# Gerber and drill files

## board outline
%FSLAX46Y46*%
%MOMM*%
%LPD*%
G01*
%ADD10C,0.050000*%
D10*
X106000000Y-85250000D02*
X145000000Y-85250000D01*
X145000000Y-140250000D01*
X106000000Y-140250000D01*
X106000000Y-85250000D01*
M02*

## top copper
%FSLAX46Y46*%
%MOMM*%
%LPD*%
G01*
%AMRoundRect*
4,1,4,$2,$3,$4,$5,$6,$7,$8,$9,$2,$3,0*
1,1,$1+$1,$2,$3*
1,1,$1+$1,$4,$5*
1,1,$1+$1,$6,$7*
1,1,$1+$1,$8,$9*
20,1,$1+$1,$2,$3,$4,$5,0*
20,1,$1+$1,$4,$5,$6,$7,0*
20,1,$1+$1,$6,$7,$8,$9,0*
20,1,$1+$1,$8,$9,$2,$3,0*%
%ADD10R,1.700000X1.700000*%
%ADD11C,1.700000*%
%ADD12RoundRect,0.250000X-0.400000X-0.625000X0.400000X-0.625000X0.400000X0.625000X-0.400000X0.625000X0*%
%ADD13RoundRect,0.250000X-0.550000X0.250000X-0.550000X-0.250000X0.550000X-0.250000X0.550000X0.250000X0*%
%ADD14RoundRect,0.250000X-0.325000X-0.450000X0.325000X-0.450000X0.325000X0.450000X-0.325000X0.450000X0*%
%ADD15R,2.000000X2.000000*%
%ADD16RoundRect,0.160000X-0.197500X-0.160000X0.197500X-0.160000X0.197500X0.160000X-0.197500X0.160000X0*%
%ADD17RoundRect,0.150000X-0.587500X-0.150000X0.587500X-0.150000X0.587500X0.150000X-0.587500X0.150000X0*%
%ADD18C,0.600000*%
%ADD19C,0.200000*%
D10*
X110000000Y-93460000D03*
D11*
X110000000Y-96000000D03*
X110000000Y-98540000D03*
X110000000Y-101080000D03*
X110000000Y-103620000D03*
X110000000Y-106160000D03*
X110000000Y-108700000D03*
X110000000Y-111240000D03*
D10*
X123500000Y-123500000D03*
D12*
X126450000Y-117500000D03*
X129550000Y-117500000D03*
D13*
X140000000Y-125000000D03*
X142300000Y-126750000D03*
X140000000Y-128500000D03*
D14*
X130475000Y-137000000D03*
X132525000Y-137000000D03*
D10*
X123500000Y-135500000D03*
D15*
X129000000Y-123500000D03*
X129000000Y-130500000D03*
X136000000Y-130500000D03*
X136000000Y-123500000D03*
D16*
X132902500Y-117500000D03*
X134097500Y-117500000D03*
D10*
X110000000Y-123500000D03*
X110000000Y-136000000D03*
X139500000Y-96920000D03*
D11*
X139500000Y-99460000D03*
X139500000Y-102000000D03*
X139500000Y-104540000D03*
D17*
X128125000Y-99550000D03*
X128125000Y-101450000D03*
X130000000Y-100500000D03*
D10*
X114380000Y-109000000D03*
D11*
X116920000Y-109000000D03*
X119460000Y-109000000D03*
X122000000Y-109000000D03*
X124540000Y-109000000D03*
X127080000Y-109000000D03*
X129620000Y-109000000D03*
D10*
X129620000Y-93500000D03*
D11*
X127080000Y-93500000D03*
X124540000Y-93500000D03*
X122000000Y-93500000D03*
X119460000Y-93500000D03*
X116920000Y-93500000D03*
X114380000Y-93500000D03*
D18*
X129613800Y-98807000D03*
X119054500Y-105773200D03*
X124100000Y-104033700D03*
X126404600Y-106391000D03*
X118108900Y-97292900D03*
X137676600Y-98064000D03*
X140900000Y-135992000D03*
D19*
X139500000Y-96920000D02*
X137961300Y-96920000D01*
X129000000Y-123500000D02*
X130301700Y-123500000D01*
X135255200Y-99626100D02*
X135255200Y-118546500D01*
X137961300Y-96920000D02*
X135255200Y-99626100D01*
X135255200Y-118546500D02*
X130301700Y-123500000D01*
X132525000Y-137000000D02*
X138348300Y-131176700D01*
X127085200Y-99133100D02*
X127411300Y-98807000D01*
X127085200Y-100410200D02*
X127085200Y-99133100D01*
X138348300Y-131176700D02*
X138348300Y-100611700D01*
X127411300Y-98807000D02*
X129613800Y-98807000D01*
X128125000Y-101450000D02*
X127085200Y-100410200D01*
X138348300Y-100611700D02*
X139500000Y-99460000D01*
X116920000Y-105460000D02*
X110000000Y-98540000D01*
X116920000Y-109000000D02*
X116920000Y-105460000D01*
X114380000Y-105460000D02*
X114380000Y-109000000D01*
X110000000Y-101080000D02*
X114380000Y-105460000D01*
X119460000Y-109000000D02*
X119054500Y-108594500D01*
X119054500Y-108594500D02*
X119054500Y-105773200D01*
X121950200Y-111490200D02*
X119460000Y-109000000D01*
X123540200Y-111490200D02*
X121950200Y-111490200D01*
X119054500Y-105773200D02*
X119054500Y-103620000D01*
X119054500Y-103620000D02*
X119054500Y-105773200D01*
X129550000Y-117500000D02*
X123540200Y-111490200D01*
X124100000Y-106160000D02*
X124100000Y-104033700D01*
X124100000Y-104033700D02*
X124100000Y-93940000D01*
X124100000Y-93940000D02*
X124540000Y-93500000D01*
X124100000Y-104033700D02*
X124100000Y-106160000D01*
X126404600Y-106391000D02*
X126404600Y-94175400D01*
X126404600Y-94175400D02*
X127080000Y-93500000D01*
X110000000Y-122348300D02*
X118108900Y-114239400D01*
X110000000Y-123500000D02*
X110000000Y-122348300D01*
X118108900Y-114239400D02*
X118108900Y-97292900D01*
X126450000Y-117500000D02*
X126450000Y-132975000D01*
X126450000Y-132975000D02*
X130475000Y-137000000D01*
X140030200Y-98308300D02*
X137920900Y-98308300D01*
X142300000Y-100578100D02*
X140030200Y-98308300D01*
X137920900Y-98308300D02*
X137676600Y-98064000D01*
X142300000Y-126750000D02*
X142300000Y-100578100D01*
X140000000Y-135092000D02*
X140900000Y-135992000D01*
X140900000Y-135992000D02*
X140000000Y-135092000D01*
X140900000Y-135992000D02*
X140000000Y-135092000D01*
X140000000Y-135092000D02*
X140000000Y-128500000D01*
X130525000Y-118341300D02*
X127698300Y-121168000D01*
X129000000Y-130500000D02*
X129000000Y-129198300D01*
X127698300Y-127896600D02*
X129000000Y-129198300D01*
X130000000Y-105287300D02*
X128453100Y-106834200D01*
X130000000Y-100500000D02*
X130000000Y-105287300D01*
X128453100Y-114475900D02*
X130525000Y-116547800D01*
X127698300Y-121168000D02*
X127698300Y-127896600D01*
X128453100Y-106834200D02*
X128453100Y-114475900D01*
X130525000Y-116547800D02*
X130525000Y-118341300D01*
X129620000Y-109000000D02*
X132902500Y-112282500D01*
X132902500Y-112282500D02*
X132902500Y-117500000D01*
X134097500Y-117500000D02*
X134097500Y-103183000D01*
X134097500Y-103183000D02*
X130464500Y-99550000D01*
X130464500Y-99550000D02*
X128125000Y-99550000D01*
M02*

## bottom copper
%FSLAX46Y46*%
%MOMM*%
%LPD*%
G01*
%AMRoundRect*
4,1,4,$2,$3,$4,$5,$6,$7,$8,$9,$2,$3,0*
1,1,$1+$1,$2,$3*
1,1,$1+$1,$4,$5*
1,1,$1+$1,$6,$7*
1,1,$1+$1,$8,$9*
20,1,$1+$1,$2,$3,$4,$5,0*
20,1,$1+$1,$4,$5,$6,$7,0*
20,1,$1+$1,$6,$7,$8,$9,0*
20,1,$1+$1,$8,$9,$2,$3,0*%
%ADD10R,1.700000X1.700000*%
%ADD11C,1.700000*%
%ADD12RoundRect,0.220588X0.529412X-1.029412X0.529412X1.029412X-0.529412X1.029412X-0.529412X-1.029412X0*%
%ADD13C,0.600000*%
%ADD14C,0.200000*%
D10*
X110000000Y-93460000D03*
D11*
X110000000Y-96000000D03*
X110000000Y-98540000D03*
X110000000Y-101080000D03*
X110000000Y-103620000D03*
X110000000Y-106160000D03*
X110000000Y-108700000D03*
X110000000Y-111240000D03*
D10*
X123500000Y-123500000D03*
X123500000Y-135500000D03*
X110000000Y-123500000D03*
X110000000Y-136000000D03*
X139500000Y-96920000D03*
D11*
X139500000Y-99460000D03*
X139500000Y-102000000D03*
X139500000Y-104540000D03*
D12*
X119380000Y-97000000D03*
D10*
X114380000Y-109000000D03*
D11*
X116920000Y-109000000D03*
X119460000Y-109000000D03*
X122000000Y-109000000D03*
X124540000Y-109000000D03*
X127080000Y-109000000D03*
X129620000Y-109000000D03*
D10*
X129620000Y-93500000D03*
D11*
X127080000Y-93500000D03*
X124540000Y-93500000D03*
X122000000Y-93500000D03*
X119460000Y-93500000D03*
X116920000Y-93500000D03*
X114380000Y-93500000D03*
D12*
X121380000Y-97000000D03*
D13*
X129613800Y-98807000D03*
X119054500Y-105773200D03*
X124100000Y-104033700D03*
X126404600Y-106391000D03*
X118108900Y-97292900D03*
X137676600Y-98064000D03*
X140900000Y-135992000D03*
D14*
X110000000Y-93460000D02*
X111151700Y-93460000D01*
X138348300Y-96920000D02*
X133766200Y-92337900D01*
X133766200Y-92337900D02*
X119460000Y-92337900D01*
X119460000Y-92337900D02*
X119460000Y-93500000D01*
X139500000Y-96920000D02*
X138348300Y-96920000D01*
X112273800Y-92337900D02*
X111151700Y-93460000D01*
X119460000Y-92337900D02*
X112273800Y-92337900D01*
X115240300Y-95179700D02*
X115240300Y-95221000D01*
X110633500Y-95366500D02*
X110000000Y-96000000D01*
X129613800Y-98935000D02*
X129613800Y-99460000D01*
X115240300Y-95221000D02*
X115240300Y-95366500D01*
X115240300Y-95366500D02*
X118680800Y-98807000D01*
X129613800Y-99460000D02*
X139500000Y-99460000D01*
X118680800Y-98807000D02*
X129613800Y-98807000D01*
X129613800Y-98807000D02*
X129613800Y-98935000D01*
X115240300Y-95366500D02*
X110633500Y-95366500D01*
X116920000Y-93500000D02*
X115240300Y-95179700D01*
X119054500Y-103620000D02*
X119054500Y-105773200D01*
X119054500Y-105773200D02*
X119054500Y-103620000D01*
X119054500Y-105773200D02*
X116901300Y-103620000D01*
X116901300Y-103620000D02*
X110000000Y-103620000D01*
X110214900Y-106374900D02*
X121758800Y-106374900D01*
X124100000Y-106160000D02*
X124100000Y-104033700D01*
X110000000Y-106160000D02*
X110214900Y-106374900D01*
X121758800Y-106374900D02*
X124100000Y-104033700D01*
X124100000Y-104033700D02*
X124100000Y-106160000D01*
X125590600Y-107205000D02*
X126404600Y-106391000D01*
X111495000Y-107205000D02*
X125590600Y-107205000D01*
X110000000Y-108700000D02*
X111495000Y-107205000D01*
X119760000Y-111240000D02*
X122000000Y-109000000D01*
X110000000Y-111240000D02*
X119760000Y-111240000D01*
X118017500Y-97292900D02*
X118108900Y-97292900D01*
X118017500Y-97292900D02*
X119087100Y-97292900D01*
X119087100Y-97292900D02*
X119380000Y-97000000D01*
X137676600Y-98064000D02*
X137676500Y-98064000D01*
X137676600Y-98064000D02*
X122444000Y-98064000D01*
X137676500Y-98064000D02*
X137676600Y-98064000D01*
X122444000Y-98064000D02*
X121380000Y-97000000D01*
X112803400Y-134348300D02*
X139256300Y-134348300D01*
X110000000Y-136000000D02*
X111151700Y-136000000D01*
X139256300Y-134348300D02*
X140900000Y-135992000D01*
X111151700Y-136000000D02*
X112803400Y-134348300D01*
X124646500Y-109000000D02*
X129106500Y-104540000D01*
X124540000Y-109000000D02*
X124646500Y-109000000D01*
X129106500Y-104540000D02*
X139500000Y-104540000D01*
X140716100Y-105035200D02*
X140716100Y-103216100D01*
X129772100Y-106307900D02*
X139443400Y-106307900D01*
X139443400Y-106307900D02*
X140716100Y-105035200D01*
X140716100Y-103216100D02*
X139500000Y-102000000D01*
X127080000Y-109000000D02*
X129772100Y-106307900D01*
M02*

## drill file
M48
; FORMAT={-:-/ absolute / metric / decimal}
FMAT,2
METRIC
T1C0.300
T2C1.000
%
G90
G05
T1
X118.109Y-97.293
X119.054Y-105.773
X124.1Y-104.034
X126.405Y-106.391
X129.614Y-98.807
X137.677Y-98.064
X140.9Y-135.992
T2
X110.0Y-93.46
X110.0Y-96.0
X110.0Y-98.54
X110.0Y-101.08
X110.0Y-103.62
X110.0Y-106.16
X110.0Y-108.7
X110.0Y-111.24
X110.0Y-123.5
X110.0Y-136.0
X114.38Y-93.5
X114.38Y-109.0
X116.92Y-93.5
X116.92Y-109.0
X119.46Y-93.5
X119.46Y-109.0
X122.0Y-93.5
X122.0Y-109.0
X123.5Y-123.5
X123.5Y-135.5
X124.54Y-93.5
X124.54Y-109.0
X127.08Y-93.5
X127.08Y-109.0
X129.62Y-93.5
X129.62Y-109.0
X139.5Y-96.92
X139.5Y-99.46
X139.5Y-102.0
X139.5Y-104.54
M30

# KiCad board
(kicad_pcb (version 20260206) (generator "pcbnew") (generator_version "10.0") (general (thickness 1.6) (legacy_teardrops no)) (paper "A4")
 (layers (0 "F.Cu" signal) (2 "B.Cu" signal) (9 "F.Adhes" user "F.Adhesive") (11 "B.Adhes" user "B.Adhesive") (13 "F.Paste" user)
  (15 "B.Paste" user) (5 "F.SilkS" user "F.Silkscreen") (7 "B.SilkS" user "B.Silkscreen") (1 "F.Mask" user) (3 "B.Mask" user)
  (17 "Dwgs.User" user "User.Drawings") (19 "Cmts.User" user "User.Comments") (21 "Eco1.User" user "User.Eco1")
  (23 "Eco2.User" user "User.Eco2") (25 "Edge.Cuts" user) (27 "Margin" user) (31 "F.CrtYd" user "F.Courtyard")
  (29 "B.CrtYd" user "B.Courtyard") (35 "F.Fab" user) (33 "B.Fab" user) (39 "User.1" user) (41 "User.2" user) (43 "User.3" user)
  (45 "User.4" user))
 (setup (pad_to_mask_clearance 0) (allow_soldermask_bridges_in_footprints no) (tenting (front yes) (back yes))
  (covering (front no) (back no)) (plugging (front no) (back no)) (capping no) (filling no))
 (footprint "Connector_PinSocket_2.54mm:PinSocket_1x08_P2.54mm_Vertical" (layer "F.Cu") (at 110 93.46)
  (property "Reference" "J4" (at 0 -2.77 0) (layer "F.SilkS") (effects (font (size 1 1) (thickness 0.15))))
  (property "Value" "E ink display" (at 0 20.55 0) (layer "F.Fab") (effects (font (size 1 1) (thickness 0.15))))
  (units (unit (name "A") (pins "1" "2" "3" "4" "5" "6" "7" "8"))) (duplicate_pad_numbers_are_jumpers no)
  (pad "1" thru_hole rect (at 0 0) (size 1.7 1.7) (drill 1) (layers "*.Cu" "*.Mask") (remove_unused_layers no) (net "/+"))
  (pad "2" thru_hole circle (at 0 2.54) (size 1.7 1.7) (drill 1) (layers "*.Cu" "*.Mask") (remove_unused_layers no) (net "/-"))
  (pad "3" thru_hole circle (at 0 5.08) (size 1.7 1.7) (drill 1) (layers "*.Cu" "*.Mask") (remove_unused_layers no) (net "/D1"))
  (pad "4" thru_hole circle (at 0 7.62) (size 1.7 1.7) (drill 1) (layers "*.Cu" "*.Mask") (remove_unused_layers no) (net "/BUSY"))
  (pad "5" thru_hole circle (at 0 10.16) (size 1.7 1.7) (drill 1) (layers "*.Cu" "*.Mask") (remove_unused_layers no) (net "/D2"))
  (pad "6" thru_hole circle (at 0 12.7) (size 1.7 1.7) (drill 1) (layers "*.Cu" "*.Mask") (remove_unused_layers no) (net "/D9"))
  (pad "7" thru_hole circle (at 0 15.24) (size 1.7 1.7) (drill 1) (layers "*.Cu" "*.Mask") (remove_unused_layers no) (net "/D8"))
  (pad "8" thru_hole circle (at 0 17.78) (size 1.7 1.7) (drill 1) (layers "*.Cu" "*.Mask") (remove_unused_layers no) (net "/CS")))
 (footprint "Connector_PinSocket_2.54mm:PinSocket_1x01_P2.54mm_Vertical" (layer "F.Cu") (at 123.5 123.5)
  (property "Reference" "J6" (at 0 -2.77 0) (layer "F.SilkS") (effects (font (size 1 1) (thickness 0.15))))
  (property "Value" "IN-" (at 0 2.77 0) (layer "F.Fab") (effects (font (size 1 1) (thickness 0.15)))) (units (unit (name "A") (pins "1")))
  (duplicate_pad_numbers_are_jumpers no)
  (pad "1" thru_hole rect (at 0 0) (size 1.7 1.7) (drill 1) (layers "*.Cu" "*.Mask") (remove_unused_layers no)
   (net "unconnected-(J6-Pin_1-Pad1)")))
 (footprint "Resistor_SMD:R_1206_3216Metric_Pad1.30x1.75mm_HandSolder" (layer "F.Cu") (at 128 117.5)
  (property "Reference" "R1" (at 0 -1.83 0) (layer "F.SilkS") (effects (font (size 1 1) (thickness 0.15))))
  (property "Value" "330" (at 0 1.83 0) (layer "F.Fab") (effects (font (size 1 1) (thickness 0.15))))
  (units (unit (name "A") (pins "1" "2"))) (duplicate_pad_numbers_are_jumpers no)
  (pad "1" smd roundrect (at -1.55 0) (size 1.3 1.75) (layers "F.Cu" "F.Mask" "F.Paste") (roundrect_rratio 0.192308) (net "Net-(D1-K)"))
  (pad "2" smd roundrect (at 1.55 0) (size 1.3 1.75) (layers "F.Cu" "F.Mask" "F.Paste") (roundrect_rratio 0.192308) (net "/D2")))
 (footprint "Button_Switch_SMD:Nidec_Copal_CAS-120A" (layer "F.Cu") (at 141.15 126.75)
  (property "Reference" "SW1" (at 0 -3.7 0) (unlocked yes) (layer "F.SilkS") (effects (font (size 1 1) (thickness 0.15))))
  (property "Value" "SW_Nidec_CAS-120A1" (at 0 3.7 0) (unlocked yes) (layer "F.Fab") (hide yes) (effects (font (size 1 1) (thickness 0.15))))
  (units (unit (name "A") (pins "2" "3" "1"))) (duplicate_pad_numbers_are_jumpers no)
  (pad "1" smd roundrect (at -1.15 -1.75 270) (size 1 1.6) (layers "F.Cu" "F.Mask" "F.Paste") (roundrect_rratio 0.25)
   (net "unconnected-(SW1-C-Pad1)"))
  (pad "2" smd roundrect (at 1.15 0 270) (size 1 1.6) (layers "F.Cu" "F.Mask" "F.Paste") (roundrect_rratio 0.25) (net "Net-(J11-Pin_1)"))
  (pad "3" smd roundrect (at -1.15 1.75 270) (size 1 1.6) (layers "F.Cu" "F.Mask" "F.Paste") (roundrect_rratio 0.25) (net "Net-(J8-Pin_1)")))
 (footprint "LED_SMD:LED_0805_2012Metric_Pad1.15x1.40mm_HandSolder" (layer "F.Cu") (at 131.5 137)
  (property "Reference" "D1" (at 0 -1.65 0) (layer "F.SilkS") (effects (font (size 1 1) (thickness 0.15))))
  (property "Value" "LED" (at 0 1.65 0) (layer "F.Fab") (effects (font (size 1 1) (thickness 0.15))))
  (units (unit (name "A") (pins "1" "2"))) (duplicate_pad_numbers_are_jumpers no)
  (pad "1" smd roundrect (at -1.025 0) (size 1.15 1.4) (layers "F.Cu" "F.Mask" "F.Paste") (roundrect_rratio 0.217391) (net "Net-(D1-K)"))
  (pad "2" smd roundrect (at 1.025 0) (size 1.15 1.4) (layers "F.Cu" "F.Mask" "F.Paste") (roundrect_rratio 0.217391) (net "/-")))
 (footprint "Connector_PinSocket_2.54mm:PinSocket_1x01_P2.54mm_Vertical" (layer "F.Cu") (at 123.5 135.5)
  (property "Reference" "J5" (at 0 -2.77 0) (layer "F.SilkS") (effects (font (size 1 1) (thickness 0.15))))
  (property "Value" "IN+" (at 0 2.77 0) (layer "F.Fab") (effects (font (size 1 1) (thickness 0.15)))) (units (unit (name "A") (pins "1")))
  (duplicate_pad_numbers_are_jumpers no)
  (pad "1" thru_hole rect (at 0 0) (size 1.7 1.7) (drill 1) (layers "*.Cu" "*.Mask") (remove_unused_layers no)
   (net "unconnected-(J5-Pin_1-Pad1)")))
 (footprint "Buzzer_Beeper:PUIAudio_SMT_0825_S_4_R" (layer "F.Cu") (at 132.5 127)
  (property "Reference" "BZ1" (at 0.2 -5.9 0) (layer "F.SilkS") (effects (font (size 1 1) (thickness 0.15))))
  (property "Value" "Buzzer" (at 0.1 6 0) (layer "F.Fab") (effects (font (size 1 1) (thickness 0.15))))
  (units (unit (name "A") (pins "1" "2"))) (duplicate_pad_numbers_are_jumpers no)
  (pad "1" smd rect (at -3.5 -3.5 270) (size 2 2) (layers "F.Cu" "F.Mask" "F.Paste") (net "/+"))
  (pad "2" smd rect (at -3.5 3.5 270) (size 2 2) (layers "F.Cu" "F.Mask" "F.Paste") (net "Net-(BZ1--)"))
  (pad "3" smd rect (at 3.5 3.5 270) (size 2 2) (layers "F.Cu" "F.Mask" "F.Paste"))
  (pad "4" smd rect (at 3.5 -3.5 270) (size 2 2) (layers "F.Cu" "F.Mask" "F.Paste")))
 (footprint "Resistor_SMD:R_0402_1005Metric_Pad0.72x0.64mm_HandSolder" (layer "F.Cu") (at 133.5 117.5)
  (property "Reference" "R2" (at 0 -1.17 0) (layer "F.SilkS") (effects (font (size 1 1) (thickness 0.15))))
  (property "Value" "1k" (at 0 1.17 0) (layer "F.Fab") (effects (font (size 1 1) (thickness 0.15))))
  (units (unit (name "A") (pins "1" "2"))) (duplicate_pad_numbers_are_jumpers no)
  (pad "1" smd roundrect (at -0.5975 0) (size 0.715 0.64) (layers "F.Cu" "F.Mask" "F.Paste") (roundrect_rratio 0.25) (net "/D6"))
  (pad "2" smd roundrect (at 0.5975 0) (size 0.715 0.64) (layers "F.Cu" "F.Mask" "F.Paste") (roundrect_rratio 0.25) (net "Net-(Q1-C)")))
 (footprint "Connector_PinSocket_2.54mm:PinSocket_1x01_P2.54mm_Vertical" (layer "F.Cu") (at 110 123.5)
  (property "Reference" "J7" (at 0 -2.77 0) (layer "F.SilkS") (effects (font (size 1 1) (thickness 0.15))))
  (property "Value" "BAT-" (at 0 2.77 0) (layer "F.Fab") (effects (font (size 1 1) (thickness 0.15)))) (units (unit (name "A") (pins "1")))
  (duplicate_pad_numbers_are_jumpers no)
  (pad "1" thru_hole rect (at 0 0) (size 1.7 1.7) (drill 1) (layers "*.Cu" "*.Mask") (remove_unused_layers no) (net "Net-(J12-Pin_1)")))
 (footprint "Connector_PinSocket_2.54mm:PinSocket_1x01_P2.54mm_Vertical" (layer "F.Cu") (at 110 136)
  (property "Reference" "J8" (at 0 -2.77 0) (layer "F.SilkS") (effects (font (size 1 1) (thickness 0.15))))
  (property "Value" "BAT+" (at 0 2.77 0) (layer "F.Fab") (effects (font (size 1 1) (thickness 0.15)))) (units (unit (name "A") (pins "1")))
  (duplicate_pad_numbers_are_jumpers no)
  (pad "1" thru_hole rect (at 0 0) (size 1.7 1.7) (drill 1) (layers "*.Cu" "*.Mask") (remove_unused_layers no) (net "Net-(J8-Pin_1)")))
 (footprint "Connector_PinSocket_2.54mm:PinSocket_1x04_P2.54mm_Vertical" (layer "F.Cu") (at 139.5 96.92)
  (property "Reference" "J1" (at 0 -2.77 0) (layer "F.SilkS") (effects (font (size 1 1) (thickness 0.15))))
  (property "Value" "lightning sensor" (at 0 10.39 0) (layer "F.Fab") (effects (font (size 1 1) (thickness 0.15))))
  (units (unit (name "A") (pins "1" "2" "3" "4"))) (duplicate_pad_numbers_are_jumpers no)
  (pad "1" thru_hole rect (at 0 0) (size 1.7 1.7) (drill 1) (layers "*.Cu" "*.Mask") (remove_unused_layers no) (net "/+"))
  (pad "2" thru_hole circle (at 0 2.54) (size 1.7 1.7) (drill 1) (layers "*.Cu" "*.Mask") (remove_unused_layers no) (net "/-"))
  (pad "3" thru_hole circle (at 0 5.08) (size 1.7 1.7) (drill 1) (layers "*.Cu" "*.Mask") (remove_unused_layers no) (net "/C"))
  (pad "4" thru_hole circle (at 0 7.62) (size 1.7 1.7) (drill 1) (layers "*.Cu" "*.Mask") (remove_unused_layers no) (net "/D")))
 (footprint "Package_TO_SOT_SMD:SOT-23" (layer "F.Cu") (at 129.0625 100.5)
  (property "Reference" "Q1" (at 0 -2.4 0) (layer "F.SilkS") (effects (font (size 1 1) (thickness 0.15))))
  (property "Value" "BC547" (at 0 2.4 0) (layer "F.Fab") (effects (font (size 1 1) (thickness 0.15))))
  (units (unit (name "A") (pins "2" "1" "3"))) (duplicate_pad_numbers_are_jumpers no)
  (pad "1" smd roundrect (at -0.9375 -0.95) (size 1.475 0.6) (layers "F.Cu" "F.Mask" "F.Paste") (roundrect_rratio 0.25) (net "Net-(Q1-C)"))
  (pad "2" smd roundrect (at -0.9375 0.95) (size 1.475 0.6) (layers "F.Cu" "F.Mask" "F.Paste") (roundrect_rratio 0.25) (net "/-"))
  (pad "3" smd roundrect (at 0.9375 0) (size 1.475 0.6) (layers "F.Cu" "F.Mask" "F.Paste") (roundrect_rratio 0.25) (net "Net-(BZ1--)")))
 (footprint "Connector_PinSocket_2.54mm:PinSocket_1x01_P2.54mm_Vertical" (layer "B.Cu") (at 119.38 97 90)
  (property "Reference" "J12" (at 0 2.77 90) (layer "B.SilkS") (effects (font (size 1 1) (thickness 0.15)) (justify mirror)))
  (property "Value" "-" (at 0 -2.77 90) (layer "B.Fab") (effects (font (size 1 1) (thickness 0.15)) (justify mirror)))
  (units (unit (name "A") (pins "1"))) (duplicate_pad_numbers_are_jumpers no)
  (pad "1" smd roundrect (at 0 0 90) (size 2.5 1.5) (layers "B.Cu" "B.Mask" "B.Paste") (roundrect_rratio 0.1470588235)
   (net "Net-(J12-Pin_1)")))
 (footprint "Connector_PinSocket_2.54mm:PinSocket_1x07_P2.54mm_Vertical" (layer "B.Cu") (at 114.38 109 -90)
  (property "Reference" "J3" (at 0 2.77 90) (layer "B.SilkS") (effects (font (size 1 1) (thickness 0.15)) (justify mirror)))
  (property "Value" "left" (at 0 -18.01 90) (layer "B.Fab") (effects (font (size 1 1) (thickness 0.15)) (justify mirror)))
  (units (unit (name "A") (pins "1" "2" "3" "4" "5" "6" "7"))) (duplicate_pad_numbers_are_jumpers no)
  (pad "1" thru_hole rect (at 0 0 270) (size 1.7 1.7) (drill 1) (layers "*.Cu" "*.Mask") (remove_unused_layers no) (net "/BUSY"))
  (pad "2" thru_hole circle (at 0 -2.54 270) (size 1.7 1.7) (drill 1) (layers "*.Cu" "*.Mask") (remove_unused_layers no) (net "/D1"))
  (pad "3" thru_hole circle (at 0 -5.08 270) (size 1.7 1.7) (drill 1) (layers "*.Cu" "*.Mask") (remove_unused_layers no) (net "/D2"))
  (pad "4" thru_hole circle (at 0 -7.62 270) (size 1.7 1.7) (drill 1) (layers "*.Cu" "*.Mask") (remove_unused_layers no) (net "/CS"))
  (pad "5" thru_hole circle (at 0 -10.16 270) (size 1.7 1.7) (drill 1) (layers "*.Cu" "*.Mask") (remove_unused_layers no) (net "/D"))
  (pad "6" thru_hole circle (at 0 -12.7 270) (size 1.7 1.7) (drill 1) (layers "*.Cu" "*.Mask") (remove_unused_layers no) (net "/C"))
  (pad "7" thru_hole circle (at 0 -15.24 270) (size 1.7 1.7) (drill 1) (layers "*.Cu" "*.Mask") (remove_unused_layers no) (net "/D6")))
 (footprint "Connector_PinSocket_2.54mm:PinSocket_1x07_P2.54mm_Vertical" (layer "B.Cu") (at 129.62 93.5 90)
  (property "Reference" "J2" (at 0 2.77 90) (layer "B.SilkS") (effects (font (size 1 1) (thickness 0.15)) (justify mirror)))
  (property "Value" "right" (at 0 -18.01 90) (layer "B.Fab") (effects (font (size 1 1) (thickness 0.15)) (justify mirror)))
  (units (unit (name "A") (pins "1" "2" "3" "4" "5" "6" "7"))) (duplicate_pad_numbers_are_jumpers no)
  (pad "1" thru_hole rect (at 0 0 90) (size 1.7 1.7) (drill 1) (layers "*.Cu" "*.Mask") (remove_unused_layers no) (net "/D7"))
  (pad "2" thru_hole circle (at 0 -2.54 90) (size 1.7 1.7) (drill 1) (layers "*.Cu" "*.Mask") (remove_unused_layers no) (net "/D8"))
  (pad "3" thru_hole circle (at 0 -5.08 90) (size 1.7 1.7) (drill 1) (layers "*.Cu" "*.Mask") (remove_unused_layers no) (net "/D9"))
  (pad "4" thru_hole circle (at 0 -7.62 90) (size 1.7 1.7) (drill 1) (layers "*.Cu" "*.Mask") (remove_unused_layers no) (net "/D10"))
  (pad "5" thru_hole circle (at 0 -10.16 90) (size 1.7 1.7) (drill 1) (layers "*.Cu" "*.Mask") (remove_unused_layers no) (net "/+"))
  (pad "6" thru_hole circle (at 0 -12.7 90) (size 1.7 1.7) (drill 1) (layers "*.Cu" "*.Mask") (remove_unused_layers no) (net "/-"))
  (pad "7" thru_hole circle (at 0 -15.24 90) (size 1.7 1.7) (drill 1) (layers "*.Cu" "*.Mask") (remove_unused_layers no) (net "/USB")))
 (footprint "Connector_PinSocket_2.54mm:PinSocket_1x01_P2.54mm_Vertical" (layer "B.Cu") (at 121.38 97 90)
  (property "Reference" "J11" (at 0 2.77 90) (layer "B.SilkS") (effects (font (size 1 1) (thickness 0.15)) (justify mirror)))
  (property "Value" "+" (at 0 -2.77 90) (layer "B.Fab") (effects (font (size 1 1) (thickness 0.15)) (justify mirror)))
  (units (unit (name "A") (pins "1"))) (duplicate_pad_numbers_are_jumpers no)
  (pad "1" smd roundrect (at 0 0 90) (size 2.5 1.5) (layers "B.Cu" "B.Mask" "B.Paste") (roundrect_rratio 0.1470588235)
   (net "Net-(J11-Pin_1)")))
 (gr_rect (start 106 85.25) (end 145 140.25) (stroke (width 0.05) (type solid)) (fill no) (layer "Edge.Cuts"))
 (segment (start 139.5 96.92) (end 137.9613 96.92) (width 0.2) (layer "F.Cu") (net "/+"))
 (segment (start 129 123.5) (end 130.3017 123.5) (width 0.2) (layer "F.Cu") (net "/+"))
 (segment (start 135.2552 99.6261) (end 135.2552 118.5465) (width 0.2) (layer "F.Cu") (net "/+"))
 (segment (start 137.9613 96.92) (end 135.2552 99.6261) (width 0.2) (layer "F.Cu") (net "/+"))
 (segment (start 135.2552 118.5465) (end 130.3017 123.5) (width 0.2) (layer "F.Cu") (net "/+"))
 (segment (start 110 93.46) (end 111.1517 93.46) (width 0.2) (layer "B.Cu") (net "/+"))
 (segment (start 138.3483 96.92) (end 133.7662 92.3379) (width 0.2) (layer "B.Cu") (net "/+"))
 (segment (start 133.7662 92.3379) (end 119.46 92.3379) (width 0.2) (layer "B.Cu") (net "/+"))
 (segment (start 119.46 92.3379) (end 119.46 93.5) (width 0.2) (layer "B.Cu") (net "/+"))
 (segment (start 139.5 96.92) (end 138.3483 96.92) (width 0.2) (layer "B.Cu") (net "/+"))
 (segment (start 112.2738 92.3379) (end 111.1517 93.46) (width 0.2) (layer "B.Cu") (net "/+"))
 (segment (start 119.46 92.3379) (end 112.2738 92.3379) (width 0.2) (layer "B.Cu") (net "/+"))
 (segment (start 132.525 137) (end 138.3483 131.1767) (width 0.2) (layer "F.Cu") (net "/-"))
 (segment (start 127.0852 99.1331) (end 127.4113 98.807) (width 0.2) (layer "F.Cu") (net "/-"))
 (segment (start 127.0852 100.4102) (end 127.0852 99.1331) (width 0.2) (layer "F.Cu") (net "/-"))
 (segment (start 138.3483 131.1767) (end 138.3483 100.6117) (width 0.2) (layer "F.Cu") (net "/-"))
 (segment (start 127.4113 98.807) (end 129.6138 98.807) (width 0.2) (layer "F.Cu") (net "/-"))
 (segment (start 128.125 101.45) (end 127.0852 100.4102) (width 0.2) (layer "F.Cu") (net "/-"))
 (segment (start 138.3483 100.6117) (end 139.5 99.46) (width 0.2) (layer "F.Cu") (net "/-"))
 (via (at 129.6138 98.807) (size 0.6) (drill 0.3) (layers "F.Cu" "B.Cu") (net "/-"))
 (segment (start 115.2403 95.1797) (end 115.2403 95.221) (width 0.2) (layer "B.Cu") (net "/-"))
 (segment (start 110.6335 95.3665) (end 110 96) (width 0.2) (layer "B.Cu") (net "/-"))
 (segment (start 129.6138 98.935) (end 129.6138 99.46) (width 0.2) (layer "B.Cu") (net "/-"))
 (segment (start 115.2403 95.221) (end 115.2403 95.3665) (width 0.2) (layer "B.Cu") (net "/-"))
 (segment (start 115.2403 95.3665) (end 118.6808 98.807) (width 0.2) (layer "B.Cu") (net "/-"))
 (segment (start 129.6138 99.46) (end 139.5 99.46) (width 0.2) (layer "B.Cu") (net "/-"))
 (segment (start 118.6808 98.807) (end 129.6138 98.807) (width 0.2) (layer "B.Cu") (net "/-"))
 (segment (start 129.6138 98.807) (end 129.6138 98.935) (width 0.2) (layer "B.Cu") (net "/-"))
 (segment (start 115.2403 95.3665) (end 110.6335 95.3665) (width 0.2) (layer "B.Cu") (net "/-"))
 (segment (start 116.92 93.5) (end 115.2403 95.1797) (width 0.2) (layer "B.Cu") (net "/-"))
 (segment (start 116.92 105.46) (end 110 98.54) (width 0.2) (layer "F.Cu") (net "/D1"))
 (segment (start 116.92 109) (end 116.92 105.46) (width 0.2) (layer "F.Cu") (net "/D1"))
 (segment (start 114.38 105.46) (end 114.38 109) (width 0.2) (layer "F.Cu") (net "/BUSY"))
 (segment (start 110 101.08) (end 114.38 105.46) (width 0.2) (layer "F.Cu") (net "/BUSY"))
 (segment (start 119.46 109) (end 119.0545 108.5945) (width 0.2) (layer "F.Cu") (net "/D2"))
 (segment (start 119.0545 108.5945) (end 119.0545 105.7732) (width 0.2) (layer "F.Cu") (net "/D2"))
 (segment (start 121.9502 111.4902) (end 119.46 109) (width 0.2) (layer "F.Cu") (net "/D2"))
 (segment (start 123.5402 111.4902) (end 121.9502 111.4902) (width 0.2) (layer "F.Cu") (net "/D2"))
 (segment (start 119.0545 105.7732) (end 119.0545 103.62) (width 0.2) (layer "F.Cu") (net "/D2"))
 (segment (start 119.0545 103.62) (end 119.0545 105.7732) (width 0.2) (layer "F.Cu") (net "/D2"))
 (segment (start 129.55 117.5) (end 123.5402 111.4902) (width 0.2) (layer "F.Cu") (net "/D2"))
 (via (at 119.0545 105.7732) (size 0.6) (drill 0.3) (layers "F.Cu" "B.Cu") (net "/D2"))
 (segment (start 119.0545 103.62) (end 119.0545 105.7732) (width 0.2) (layer "B.Cu") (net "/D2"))
 (segment (start 119.0545 105.7732) (end 119.0545 103.62) (width 0.2) (layer "B.Cu") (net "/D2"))
 (segment (start 119.0545 105.7732) (end 116.9013 103.62) (width 0.2) (layer "B.Cu") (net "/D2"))
 (segment (start 116.9013 103.62) (end 110 103.62) (width 0.2) (layer "B.Cu") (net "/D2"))
 (segment (start 124.1 106.16) (end 124.1 104.0337) (width 0.2) (layer "F.Cu") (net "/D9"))
 (segment (start 124.1 104.0337) (end 124.1 93.94) (width 0.2) (layer "F.Cu") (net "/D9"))
 (segment (start 124.1 93.94) (end 124.54 93.5) (width 0.2) (layer "F.Cu") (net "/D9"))
 (segment (start 124.1 104.0337) (end 124.1 106.16) (width 0.2) (layer "F.Cu") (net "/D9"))
 (via (at 124.1 104.0337) (size 0.6) (drill 0.3) (layers "F.Cu" "B.Cu") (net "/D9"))
 (segment (start 110.2149 106.3749) (end 121.7588 106.3749) (width 0.2) (layer "B.Cu") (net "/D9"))
 (segment (start 124.1 106.16) (end 124.1 104.0337) (width 0.2) (layer "B.Cu") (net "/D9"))
 (segment (start 110 106.16) (end 110.2149 106.3749) (width 0.2) (layer "B.Cu") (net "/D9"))
 (segment (start 121.7588 106.3749) (end 124.1 104.0337) (width 0.2) (layer "B.Cu") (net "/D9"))
 (segment (start 124.1 104.0337) (end 124.1 106.16) (width 0.2) (layer "B.Cu") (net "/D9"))
 (segment (start 126.4046 106.391) (end 126.4046 94.1754) (width 0.2) (layer "F.Cu") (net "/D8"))
 (segment (start 126.4046 94.1754) (end 127.08 93.5) (width 0.2) (layer "F.Cu") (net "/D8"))
 (via (at 126.4046 106.391) (size 0.6) (drill 0.3) (layers "F.Cu" "B.Cu") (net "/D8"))
 (segment (start 125.5906 107.205) (end 126.4046 106.391) (width 0.2) (layer "B.Cu") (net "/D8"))
 (segment (start 111.495 107.205) (end 125.5906 107.205) (width 0.2) (layer "B.Cu") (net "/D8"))
 (segment (start 110 108.7) (end 111.495 107.205) (width 0.2) (layer "B.Cu") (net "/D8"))
 (segment (start 119.76 111.24) (end 122 109) (width 0.2) (layer "B.Cu") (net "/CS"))
 (segment (start 110 111.24) (end 119.76 111.24) (width 0.2) (layer "B.Cu") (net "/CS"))
 (segment (start 110 122.3483) (end 118.1089 114.2394) (width 0.2) (layer "F.Cu") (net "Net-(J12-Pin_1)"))
 (segment (start 110 123.5) (end 110 122.3483) (width 0.2) (layer "F.Cu") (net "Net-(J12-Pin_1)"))
 (segment (start 118.1089 114.2394) (end 118.1089 97.2929) (width 0.2) (layer "F.Cu") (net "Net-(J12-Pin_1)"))
 (via (at 118.1089 97.2929) (size 0.6) (drill 0.3) (layers "F.Cu" "B.Cu") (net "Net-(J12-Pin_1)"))
 (segment (start 118.0175 97.2929) (end 118.1089 97.2929) (width 0.2) (layer "B.Cu") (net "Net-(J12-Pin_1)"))
 (segment (start 118.0175 97.2929) (end 119.0871 97.2929) (width 0.2) (layer "B.Cu") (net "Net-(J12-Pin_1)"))
 (segment (start 119.0871 97.2929) (end 119.38 97) (width 0.2) (layer "B.Cu") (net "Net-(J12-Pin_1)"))
 (segment (start 126.45 117.5) (end 126.45 132.975) (width 0.2) (layer "F.Cu") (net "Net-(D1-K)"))
 (segment (start 126.45 132.975) (end 130.475 137) (width 0.2) (layer "F.Cu") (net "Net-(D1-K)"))
 (segment (start 140.0302 98.3083) (end 137.9209 98.3083) (width 0.2) (layer "F.Cu") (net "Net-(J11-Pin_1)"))
 (segment (start 142.3 100.5781) (end 140.0302 98.3083) (width 0.2) (layer "F.Cu") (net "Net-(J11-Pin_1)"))
 (segment (start 137.9209 98.3083) (end 137.6766 98.064) (width 0.2) (layer "F.Cu") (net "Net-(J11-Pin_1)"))
 (segment (start 142.3 126.75) (end 142.3 100.5781) (width 0.2) (layer "F.Cu") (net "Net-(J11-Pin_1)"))
 (via (at 137.6766 98.064) (size 0.6) (drill 0.3) (layers "F.Cu" "B.Cu") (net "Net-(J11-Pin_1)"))
 (segment (start 137.6766 98.064) (end 137.6765 98.064) (width 0.2) (layer "B.Cu") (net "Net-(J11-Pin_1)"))
 (segment (start 137.6766 98.064) (end 122.444 98.064) (width 0.2) (layer "B.Cu") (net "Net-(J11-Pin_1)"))
 (segment (start 137.6765 98.064) (end 137.6766 98.064) (width 0.2) (layer "B.Cu") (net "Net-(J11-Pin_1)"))
 (segment (start 122.444 98.064) (end 121.38 97) (width 0.2) (layer "B.Cu") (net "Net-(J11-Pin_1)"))
 (segment (start 140 135.092) (end 140.9 135.992) (width 0.2) (layer "F.Cu") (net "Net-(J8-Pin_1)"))
 (segment (start 140.9 135.992) (end 140 135.092) (width 0.2) (layer "F.Cu") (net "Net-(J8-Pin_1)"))
 (segment (start 140.9 135.992) (end 140 135.092) (width 0.2) (layer "F.Cu") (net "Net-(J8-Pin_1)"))
 (segment (start 140 135.092) (end 140 128.5) (width 0.2) (layer "F.Cu") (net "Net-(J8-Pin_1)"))
 (via (at 140.9 135.992) (size 0.6) (drill 0.3) (layers "F.Cu" "B.Cu") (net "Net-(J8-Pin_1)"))
 (segment (start 112.8034 134.3483) (end 139.2563 134.3483) (width 0.2) (layer "B.Cu") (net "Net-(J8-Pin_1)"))
 (segment (start 110 136) (end 111.1517 136) (width 0.2) (layer "B.Cu") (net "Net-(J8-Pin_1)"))
 (segment (start 139.2563 134.3483) (end 140.9 135.992) (width 0.2) (layer "B.Cu") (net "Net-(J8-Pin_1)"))
 (segment (start 111.1517 136) (end 112.8034 134.3483) (width 0.2) (layer "B.Cu") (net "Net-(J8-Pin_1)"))
 (segment (start 130.525 118.3413) (end 127.6983 121.168) (width 0.2) (layer "F.Cu") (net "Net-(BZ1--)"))
 (segment (start 129 130.5) (end 129 129.1983) (width 0.2) (layer "F.Cu") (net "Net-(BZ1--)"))
 (segment (start 127.6983 127.8966) (end 129 129.1983) (width 0.2) (layer "F.Cu") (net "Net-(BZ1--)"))
 (segment (start 130 105.2873) (end 128.4531 106.8342) (width 0.2) (layer "F.Cu") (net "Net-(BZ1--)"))
 (segment (start 130 100.5) (end 130 105.2873) (width 0.2) (layer "F.Cu") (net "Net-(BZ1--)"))
 (segment (start 128.4531 114.4759) (end 130.525 116.5478) (width 0.2) (layer "F.Cu") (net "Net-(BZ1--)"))
 (segment (start 127.6983 121.168) (end 127.6983 127.8966) (width 0.2) (layer "F.Cu") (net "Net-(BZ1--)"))
 (segment (start 128.4531 106.8342) (end 128.4531 114.4759) (width 0.2) (layer "F.Cu") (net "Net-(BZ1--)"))
 (segment (start 130.525 116.5478) (end 130.525 118.3413) (width 0.2) (layer "F.Cu") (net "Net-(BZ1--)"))
 (segment (start 129.62 109) (end 132.9025 112.2825) (width 0.2) (layer "F.Cu") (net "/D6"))
 (segment (start 132.9025 112.2825) (end 132.9025 117.5) (width 0.2) (layer "F.Cu") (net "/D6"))
 (segment (start 134.0975 117.5) (end 134.0975 103.183) (width 0.2) (layer "F.Cu") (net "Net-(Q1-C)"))
 (segment (start 134.0975 103.183) (end 130.4645 99.55) (width 0.2) (layer "F.Cu") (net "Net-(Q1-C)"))
 (segment (start 130.4645 99.55) (end 128.125 99.55) (width 0.2) (layer "F.Cu") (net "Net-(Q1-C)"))
 (segment (start 124.6465 109) (end 129.1065 104.54) (width 0.2) (layer "B.Cu") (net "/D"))
 (segment (start 124.54 109) (end 124.6465 109) (width 0.2) (layer "B.Cu") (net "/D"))
 (segment (start 129.1065 104.54) (end 139.5 104.54) (width 0.2) (layer "B.Cu") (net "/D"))
 (segment (start 140.7161 105.0352) (end 140.7161 103.2161) (width 0.2) (layer "B.Cu") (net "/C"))
 (segment (start 129.7721 106.3079) (end 139.4434 106.3079) (width 0.2) (layer "B.Cu") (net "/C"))
 (segment (start 139.4434 106.3079) (end 140.7161 105.0352) (width 0.2) (layer "B.Cu") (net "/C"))
 (segment (start 140.7161 103.2161) (end 139.5 102) (width 0.2) (layer "B.Cu") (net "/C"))
 (segment (start 127.08 109) (end 129.7721 106.3079) (width 0.2) (layer "B.Cu") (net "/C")))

